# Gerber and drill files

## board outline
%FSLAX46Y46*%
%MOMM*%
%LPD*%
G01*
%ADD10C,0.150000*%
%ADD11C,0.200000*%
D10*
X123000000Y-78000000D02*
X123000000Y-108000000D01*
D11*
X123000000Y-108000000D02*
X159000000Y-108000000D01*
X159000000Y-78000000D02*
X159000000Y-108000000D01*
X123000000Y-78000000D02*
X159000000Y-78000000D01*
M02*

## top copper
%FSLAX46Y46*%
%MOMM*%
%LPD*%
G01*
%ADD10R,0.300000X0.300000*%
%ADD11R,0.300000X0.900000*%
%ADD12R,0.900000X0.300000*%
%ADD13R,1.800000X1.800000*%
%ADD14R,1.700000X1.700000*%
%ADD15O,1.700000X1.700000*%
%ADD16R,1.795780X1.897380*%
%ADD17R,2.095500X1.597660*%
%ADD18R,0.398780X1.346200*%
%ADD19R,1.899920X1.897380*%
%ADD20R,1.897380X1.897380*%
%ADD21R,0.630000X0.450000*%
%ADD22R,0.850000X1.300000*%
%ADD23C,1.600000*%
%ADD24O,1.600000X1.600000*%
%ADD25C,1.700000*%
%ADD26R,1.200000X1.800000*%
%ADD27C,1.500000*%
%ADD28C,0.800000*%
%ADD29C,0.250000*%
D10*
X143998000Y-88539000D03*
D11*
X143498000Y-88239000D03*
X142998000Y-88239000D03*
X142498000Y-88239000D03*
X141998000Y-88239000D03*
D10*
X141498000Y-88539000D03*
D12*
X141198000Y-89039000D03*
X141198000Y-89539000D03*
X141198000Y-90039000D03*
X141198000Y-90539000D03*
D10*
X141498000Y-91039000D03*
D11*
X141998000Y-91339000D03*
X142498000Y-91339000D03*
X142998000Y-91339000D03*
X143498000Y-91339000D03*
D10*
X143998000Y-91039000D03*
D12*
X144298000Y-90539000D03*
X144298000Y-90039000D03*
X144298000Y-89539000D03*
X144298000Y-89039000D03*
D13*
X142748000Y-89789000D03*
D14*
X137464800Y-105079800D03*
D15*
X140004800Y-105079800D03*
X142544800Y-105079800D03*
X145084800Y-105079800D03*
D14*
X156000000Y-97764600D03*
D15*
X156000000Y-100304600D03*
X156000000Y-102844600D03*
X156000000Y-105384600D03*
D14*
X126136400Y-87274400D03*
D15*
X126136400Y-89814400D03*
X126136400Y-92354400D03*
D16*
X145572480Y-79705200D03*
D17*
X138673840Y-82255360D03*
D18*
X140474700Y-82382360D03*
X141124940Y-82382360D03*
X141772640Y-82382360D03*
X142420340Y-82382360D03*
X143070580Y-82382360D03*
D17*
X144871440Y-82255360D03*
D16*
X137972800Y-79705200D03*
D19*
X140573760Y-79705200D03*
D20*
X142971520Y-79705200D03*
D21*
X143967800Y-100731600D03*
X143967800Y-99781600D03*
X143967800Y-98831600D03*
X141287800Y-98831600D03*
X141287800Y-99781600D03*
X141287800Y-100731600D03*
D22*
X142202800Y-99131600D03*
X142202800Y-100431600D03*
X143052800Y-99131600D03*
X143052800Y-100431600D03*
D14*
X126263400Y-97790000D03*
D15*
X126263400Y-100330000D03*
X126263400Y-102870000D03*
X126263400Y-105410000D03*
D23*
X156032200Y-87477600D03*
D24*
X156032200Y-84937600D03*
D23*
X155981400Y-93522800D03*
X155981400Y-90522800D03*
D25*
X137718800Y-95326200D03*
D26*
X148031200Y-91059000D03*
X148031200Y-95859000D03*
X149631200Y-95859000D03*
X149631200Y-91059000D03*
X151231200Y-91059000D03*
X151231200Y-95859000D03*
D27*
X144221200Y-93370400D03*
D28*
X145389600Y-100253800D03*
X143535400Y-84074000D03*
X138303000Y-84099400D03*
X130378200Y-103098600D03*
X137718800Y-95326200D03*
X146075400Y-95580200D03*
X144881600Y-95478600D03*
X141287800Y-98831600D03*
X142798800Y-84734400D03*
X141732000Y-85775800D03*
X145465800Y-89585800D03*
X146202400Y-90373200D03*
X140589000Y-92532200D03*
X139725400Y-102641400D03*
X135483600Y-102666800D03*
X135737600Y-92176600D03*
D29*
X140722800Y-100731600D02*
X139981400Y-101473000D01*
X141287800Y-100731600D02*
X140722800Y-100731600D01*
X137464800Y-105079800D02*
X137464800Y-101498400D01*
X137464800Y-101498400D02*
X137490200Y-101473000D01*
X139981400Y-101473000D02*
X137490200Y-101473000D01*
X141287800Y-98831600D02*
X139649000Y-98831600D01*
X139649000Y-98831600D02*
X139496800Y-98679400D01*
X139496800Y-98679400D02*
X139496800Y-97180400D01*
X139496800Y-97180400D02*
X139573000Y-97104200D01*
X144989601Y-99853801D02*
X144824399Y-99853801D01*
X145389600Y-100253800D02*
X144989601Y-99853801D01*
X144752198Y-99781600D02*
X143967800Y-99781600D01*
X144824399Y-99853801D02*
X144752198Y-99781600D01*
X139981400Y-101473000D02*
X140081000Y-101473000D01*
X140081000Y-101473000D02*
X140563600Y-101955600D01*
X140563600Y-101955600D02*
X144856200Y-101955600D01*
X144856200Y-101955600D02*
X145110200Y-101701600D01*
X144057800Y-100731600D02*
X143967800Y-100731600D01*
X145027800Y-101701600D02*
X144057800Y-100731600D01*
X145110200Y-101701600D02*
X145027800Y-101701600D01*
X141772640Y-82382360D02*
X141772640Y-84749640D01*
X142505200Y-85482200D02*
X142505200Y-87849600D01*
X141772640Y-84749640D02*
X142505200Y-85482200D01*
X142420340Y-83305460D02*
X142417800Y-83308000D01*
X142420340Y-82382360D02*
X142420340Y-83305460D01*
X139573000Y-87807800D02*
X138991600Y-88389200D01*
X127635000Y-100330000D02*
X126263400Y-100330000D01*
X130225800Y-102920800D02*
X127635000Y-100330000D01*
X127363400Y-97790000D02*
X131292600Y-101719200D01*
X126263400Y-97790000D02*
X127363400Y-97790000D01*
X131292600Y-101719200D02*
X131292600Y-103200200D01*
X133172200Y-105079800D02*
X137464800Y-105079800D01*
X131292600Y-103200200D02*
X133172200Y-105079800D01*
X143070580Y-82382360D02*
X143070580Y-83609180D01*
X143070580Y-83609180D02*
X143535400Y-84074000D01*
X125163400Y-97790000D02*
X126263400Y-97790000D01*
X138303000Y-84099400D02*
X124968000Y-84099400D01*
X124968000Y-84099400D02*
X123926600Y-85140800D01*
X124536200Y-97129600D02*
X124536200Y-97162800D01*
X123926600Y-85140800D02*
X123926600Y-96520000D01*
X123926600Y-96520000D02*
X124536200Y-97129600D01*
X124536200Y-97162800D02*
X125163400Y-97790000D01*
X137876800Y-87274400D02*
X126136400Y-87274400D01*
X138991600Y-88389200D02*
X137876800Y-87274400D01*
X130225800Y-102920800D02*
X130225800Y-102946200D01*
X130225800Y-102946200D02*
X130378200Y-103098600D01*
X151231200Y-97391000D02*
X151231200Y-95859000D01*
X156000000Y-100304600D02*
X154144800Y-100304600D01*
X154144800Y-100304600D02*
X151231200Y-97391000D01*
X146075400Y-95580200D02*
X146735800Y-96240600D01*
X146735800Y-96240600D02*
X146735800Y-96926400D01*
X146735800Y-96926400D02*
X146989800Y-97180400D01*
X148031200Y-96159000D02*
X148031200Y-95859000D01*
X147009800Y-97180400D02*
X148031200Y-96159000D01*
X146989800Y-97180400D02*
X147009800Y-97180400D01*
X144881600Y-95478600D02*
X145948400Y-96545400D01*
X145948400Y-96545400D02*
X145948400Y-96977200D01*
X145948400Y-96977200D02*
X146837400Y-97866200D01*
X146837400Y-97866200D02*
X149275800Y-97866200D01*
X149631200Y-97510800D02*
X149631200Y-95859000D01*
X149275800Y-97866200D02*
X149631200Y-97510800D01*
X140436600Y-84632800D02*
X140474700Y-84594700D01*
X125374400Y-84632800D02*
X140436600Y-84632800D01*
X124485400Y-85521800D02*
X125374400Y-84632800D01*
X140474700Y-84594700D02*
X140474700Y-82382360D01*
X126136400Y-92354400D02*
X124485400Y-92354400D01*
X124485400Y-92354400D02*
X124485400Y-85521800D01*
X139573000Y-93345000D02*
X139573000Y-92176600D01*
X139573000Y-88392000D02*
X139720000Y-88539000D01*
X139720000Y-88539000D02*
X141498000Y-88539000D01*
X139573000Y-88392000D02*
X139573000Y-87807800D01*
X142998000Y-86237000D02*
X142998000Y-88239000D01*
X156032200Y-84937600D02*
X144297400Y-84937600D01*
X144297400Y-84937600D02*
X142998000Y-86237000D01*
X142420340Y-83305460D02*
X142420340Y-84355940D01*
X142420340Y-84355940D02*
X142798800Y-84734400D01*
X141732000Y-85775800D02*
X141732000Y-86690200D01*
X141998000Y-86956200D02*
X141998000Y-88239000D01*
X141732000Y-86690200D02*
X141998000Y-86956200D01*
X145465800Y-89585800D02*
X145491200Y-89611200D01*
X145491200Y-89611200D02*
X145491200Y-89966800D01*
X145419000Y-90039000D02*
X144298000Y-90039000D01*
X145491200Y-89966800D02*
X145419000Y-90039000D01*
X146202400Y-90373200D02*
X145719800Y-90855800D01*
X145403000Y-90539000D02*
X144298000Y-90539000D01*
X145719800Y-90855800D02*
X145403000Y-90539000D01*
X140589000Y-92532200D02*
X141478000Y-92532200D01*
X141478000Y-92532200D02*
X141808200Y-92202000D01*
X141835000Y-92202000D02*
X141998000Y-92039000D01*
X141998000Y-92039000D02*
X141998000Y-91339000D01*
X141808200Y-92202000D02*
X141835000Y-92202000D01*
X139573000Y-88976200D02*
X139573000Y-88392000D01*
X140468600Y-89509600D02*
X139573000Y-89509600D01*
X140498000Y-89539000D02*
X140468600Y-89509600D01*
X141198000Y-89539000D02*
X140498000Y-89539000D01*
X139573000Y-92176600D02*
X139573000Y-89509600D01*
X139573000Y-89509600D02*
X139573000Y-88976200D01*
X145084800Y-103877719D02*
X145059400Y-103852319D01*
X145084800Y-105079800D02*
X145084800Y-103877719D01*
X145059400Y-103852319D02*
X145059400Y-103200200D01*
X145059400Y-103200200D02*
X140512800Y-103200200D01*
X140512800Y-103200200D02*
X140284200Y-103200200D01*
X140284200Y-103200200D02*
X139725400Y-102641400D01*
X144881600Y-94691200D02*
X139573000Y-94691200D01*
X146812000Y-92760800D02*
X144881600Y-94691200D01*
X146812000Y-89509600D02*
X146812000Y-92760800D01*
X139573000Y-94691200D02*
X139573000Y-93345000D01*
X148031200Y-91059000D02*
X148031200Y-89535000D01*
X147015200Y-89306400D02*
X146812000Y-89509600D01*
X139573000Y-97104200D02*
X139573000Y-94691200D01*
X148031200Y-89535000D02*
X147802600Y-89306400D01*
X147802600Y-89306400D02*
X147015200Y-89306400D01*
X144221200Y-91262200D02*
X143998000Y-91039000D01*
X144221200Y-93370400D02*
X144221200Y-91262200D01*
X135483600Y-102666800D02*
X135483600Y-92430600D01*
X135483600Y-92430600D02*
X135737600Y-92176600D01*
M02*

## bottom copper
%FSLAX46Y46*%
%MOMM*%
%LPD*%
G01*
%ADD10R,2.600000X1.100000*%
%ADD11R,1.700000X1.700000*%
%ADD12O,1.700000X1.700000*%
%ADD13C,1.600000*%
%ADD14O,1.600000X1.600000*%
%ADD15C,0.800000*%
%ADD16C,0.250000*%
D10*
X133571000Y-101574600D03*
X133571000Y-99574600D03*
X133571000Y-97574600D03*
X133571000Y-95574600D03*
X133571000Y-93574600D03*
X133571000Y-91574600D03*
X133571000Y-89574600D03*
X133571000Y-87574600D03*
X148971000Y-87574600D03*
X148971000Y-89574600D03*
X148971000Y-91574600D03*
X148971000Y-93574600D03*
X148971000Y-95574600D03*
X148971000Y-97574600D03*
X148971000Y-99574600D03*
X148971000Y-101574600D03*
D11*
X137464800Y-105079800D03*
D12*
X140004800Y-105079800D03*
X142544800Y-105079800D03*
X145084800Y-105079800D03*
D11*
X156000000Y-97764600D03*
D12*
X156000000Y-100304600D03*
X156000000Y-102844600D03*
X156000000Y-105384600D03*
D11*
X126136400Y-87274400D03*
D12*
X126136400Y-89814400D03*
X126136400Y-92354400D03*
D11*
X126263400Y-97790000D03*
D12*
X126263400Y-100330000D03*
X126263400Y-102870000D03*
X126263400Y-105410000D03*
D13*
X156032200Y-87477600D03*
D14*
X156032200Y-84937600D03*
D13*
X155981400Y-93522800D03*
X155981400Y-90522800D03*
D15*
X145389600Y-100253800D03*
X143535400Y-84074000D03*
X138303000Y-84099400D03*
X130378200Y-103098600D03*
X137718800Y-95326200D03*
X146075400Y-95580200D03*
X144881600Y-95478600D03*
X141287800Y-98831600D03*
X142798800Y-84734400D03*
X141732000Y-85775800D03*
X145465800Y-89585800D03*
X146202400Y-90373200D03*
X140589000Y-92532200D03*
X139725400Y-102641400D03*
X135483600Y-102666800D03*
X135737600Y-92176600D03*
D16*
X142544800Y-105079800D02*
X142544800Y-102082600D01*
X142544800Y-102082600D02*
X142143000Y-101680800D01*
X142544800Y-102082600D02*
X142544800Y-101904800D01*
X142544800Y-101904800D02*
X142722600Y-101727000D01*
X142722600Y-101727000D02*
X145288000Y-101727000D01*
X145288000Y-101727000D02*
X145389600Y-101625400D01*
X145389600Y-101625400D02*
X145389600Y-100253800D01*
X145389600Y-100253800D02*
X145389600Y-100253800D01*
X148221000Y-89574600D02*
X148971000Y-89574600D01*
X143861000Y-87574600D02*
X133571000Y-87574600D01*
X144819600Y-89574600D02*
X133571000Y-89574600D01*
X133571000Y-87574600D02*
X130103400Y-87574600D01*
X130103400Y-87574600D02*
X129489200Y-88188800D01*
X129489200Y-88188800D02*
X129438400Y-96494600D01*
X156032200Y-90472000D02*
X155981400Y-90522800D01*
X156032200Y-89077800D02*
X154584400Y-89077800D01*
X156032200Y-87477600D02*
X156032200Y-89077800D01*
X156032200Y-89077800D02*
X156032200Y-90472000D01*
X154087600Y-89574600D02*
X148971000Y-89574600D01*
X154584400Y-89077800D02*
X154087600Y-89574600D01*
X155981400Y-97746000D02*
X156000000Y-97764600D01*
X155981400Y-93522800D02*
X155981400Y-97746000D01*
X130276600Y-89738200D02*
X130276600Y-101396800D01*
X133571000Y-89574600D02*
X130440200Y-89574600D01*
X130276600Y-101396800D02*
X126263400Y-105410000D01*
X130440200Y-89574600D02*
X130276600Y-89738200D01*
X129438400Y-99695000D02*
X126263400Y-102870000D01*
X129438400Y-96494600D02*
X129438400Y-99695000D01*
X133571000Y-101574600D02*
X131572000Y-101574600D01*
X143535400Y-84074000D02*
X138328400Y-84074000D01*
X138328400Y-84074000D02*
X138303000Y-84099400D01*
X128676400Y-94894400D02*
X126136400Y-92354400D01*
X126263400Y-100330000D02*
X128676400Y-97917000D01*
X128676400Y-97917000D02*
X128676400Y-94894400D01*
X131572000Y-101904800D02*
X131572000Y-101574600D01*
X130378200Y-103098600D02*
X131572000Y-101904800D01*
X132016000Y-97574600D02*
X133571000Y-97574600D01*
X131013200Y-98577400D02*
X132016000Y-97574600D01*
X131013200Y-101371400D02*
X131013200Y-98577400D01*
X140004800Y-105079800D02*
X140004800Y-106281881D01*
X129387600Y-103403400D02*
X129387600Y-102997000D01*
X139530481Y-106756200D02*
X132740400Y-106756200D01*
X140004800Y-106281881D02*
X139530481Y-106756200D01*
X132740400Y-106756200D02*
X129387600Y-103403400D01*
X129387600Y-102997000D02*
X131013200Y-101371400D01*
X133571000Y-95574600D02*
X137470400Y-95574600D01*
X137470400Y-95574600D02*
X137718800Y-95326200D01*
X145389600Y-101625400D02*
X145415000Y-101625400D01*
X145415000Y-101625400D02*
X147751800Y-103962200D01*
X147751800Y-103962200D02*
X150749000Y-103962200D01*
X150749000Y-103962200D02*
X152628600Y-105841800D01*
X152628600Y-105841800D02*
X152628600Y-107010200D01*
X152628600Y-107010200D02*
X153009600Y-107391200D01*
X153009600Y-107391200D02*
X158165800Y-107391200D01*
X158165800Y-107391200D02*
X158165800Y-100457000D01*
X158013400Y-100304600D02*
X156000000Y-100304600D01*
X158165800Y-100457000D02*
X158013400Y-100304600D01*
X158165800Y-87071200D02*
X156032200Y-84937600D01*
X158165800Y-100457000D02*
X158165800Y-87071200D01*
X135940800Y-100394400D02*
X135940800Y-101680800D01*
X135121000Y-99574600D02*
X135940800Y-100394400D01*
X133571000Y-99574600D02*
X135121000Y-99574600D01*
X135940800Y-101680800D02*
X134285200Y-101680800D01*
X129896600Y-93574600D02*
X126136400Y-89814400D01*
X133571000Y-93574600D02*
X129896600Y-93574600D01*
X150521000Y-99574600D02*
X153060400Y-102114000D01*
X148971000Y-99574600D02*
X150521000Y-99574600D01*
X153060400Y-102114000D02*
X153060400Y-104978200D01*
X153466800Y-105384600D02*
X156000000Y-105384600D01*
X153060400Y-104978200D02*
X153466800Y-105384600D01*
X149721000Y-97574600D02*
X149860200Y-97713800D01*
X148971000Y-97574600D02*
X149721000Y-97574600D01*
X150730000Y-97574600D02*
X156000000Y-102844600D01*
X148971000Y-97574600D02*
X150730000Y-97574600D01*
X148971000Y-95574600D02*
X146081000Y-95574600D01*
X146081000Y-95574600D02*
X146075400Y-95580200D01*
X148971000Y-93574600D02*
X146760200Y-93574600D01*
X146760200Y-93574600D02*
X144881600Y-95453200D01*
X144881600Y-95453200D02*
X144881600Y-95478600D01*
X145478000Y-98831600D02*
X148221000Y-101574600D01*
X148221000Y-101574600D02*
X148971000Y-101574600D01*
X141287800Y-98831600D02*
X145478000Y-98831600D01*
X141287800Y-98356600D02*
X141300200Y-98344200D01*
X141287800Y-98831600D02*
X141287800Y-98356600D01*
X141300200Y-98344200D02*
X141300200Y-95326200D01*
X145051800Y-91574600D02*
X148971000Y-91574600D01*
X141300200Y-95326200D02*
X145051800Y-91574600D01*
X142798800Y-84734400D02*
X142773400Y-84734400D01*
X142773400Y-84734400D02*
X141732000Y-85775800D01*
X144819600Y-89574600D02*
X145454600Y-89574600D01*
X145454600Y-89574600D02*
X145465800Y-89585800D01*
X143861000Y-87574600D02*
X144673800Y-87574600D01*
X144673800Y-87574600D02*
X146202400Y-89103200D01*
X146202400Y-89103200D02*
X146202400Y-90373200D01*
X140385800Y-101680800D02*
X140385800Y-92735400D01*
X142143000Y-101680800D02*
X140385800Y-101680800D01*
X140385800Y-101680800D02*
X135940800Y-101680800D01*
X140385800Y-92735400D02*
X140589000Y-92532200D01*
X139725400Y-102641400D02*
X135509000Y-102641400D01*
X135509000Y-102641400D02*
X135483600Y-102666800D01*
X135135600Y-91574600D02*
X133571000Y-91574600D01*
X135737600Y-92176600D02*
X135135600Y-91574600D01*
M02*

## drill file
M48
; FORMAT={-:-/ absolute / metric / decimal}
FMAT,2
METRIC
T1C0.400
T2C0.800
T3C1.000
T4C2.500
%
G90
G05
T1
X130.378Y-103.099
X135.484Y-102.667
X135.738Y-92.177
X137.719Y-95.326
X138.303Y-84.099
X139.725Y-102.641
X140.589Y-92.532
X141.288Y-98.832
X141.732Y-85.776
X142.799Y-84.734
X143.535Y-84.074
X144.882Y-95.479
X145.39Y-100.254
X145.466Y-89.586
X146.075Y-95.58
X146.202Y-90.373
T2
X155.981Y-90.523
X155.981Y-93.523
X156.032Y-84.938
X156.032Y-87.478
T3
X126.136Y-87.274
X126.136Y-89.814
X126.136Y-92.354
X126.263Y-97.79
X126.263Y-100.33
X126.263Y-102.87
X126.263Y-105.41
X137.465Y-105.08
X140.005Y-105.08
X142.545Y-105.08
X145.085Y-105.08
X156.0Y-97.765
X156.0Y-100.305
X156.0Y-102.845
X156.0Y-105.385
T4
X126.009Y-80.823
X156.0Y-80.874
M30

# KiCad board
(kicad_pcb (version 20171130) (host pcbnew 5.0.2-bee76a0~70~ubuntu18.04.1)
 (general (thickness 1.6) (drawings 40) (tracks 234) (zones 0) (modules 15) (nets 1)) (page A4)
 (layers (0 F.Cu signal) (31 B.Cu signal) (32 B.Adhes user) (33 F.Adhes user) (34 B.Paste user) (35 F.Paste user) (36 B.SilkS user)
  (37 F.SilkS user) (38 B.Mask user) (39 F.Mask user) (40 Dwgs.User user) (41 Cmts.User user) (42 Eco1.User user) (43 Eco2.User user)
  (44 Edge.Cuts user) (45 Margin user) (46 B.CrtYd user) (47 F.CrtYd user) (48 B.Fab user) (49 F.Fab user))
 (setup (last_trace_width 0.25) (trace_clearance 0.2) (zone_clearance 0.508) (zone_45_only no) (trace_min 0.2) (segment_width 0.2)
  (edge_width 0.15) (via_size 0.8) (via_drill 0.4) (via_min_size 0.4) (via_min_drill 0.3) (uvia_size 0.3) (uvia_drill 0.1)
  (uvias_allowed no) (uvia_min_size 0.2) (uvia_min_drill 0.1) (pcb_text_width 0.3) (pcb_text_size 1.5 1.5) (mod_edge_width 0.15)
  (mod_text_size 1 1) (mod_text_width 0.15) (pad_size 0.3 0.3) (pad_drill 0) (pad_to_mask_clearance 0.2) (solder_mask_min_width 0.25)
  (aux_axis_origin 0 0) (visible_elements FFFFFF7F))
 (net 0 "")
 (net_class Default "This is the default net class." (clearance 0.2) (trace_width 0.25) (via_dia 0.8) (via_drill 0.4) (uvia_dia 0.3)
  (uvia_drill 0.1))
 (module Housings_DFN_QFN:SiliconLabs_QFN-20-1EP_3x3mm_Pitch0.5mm (layer F.Cu) (at 142.748 89.789 270)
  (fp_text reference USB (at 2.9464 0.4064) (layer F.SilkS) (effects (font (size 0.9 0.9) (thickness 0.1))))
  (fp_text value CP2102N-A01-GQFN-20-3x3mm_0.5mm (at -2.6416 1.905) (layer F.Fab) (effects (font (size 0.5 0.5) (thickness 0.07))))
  (pad 1 smd rect (at -1.25 -1.25 270) (size 0.3 0.3) (layers F.Cu F.Paste F.Mask))
  (pad 2 smd rect (at -1.55 -0.75 270) (size 0.9 0.3) (layers F.Cu F.Paste F.Mask))
  (pad GND smd rect (at -1.55 -0.25 270) (size 0.9 0.3) (layers F.Cu F.Paste F.Mask))
  (pad D+ smd rect (at -1.55 0.25 270) (size 0.9 0.3) (layers F.Cu F.Paste F.Mask))
  (pad D- smd rect (at -1.55 0.75 270) (size 0.9 0.3) (layers F.Cu F.Paste F.Mask))
  (pad +3.3 smd rect (at -1.25 1.25 270) (size 0.3 0.3) (layers F.Cu F.Paste F.Mask))
  (pad VREGIN smd rect (at -0.75 1.55) (size 0.9 0.3) (layers F.Cu F.Paste F.Mask))
  (pad VBUS smd rect (at -0.25 1.55) (size 0.9 0.3) (layers F.Cu F.Paste F.Mask))
  (pad 9 smd rect (at 0.25 1.55) (size 0.9 0.3) (layers F.Cu F.Paste F.Mask))
  (pad 10 smd rect (at 0.75 1.55) (size 0.9 0.3) (layers F.Cu F.Paste F.Mask))
  (pad 11 smd rect (at 1.25 1.25 270) (size 0.3 0.3) (layers F.Cu F.Paste F.Mask))
  (pad GND smd rect (at 1.55 0.75 270) (size 0.9 0.3) (layers F.Cu F.Paste F.Mask))
  (pad 13 smd rect (at 1.55 0.25 270) (size 0.9 0.3) (layers F.Cu F.Paste F.Mask))
  (pad 14 smd rect (at 1.55 -0.25 270) (size 0.9 0.3) (layers F.Cu F.Paste F.Mask))
  (pad 15 smd rect (at 1.55 -0.75 270) (size 0.9 0.3) (layers F.Cu F.Paste F.Mask))
  (pad 16 smd rect (at 1.25 -1.25 270) (size 0.3 0.3) (layers F.Cu F.Paste F.Mask))
  (pad RX smd rect (at 0.75 -1.55) (size 0.9 0.3) (layers F.Cu F.Paste F.Mask))
  (pad TX smd rect (at 0.25 -1.55) (size 0.9 0.3) (layers F.Cu F.Paste F.Mask))
  (pad 19 smd rect (at -0.25 -1.55) (size 0.9 0.3) (layers F.Cu F.Paste F.Mask))
  (pad 20 smd rect (at -0.75 -1.55) (size 0.9 0.3) (layers F.Cu F.Paste F.Mask))
  (pad 21 smd rect (at 0 0 270) (size 1.8 1.8) (layers F.Cu F.Mask))
  (pad "" smd rect (at -0.45 -0.45 270) (size 0.54 0.54) (layers F.Paste))
  (pad "" smd rect (at -0.45 0.45 270) (size 0.54 0.54) (layers F.Paste))
  (pad "" smd rect (at 0.45 -0.45 270) (size 0.54 0.54) (layers F.Paste))
  (pad "" smd rect (at 0.45 0.45 270) (size 0.54 0.54) (layers F.Paste)))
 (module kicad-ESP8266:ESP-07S (layer B.Cu) (at 141.271 94.5746)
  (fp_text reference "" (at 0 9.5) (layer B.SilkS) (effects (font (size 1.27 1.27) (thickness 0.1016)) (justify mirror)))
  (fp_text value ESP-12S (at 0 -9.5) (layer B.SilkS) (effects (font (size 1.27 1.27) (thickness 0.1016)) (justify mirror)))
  (pad GND smd rect (at -7.7 7) (size 2.6 1.1) (layers B.Cu B.Paste B.Mask))
  (pad IO15 smd rect (at -7.7 5) (size 2.6 1.1) (layers B.Cu B.Paste B.Mask))
  (pad IO2 smd rect (at -7.7 3) (size 2.6 1.1) (layers B.Cu B.Paste B.Mask))
  (pad IO0 smd rect (at -7.7 1) (size 2.6 1.1) (layers B.Cu B.Paste B.Mask))
  (pad IO4 smd rect (at -7.7 -1) (size 2.6 1.1) (layers B.Cu B.Paste B.Mask))
  (pad IO5 smd rect (at -7.7 -3) (size 2.6 1.1) (layers B.Cu B.Paste B.Mask))
  (pad RX smd rect (at -7.7 -5) (size 2.6 1.1) (layers B.Cu B.Paste B.Mask))
  (pad TX smd rect (at -7.7 -7) (size 2.6 1.1) (layers B.Cu B.Paste B.Mask))
  (pad RST smd rect (at 7.7 -7) (size 2.6 1.1) (layers B.Cu B.Paste B.Mask))
  (pad ADC smd rect (at 7.7 -5) (size 2.6 1.1) (layers B.Cu B.Paste B.Mask))
  (pad EN smd rect (at 7.7 -3) (size 2.6 1.1) (layers B.Cu B.Paste B.Mask))
  (pad IO16 smd rect (at 7.7 -1) (size 2.6 1.1) (layers B.Cu B.Paste B.Mask))
  (pad IO14 smd rect (at 7.7 1) (size 2.6 1.1) (layers B.Cu B.Paste B.Mask))
  (pad IO12 smd rect (at 7.7 3) (size 2.6 1.1) (layers B.Cu B.Paste B.Mask))
  (pad IO13 smd rect (at 7.7 5) (size 2.6 1.1) (layers B.Cu B.Paste B.Mask))
  (pad VCC smd rect (at 7.7 7) (size 2.6 1.1) (layers B.Cu B.Paste B.Mask)))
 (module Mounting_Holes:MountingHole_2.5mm (layer F.Cu) (at 126.0094 80.8228)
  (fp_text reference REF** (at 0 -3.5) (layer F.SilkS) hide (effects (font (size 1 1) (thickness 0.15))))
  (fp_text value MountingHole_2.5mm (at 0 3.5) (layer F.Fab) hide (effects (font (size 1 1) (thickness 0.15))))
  (pad 1 np_thru_hole circle (at 0 0) (size 2.5 2.5) (drill 2.5) (layers *.Cu *.Mask)))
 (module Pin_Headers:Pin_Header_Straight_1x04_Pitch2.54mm (layer F.Cu) (at 137.4648 105.0798 90)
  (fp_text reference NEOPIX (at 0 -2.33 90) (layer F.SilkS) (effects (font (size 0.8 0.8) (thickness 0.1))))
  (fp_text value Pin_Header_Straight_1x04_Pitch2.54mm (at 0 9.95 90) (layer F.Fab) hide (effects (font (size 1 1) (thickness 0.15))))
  (pad +V thru_hole rect (at 0 0 90) (size 1.7 1.7) (drill 1) (layers *.Cu *.Mask))
  (pad 2 thru_hole oval (at 0 2.54 90) (size 1.7 1.7) (drill 1) (layers *.Cu *.Mask))
  (pad GND thru_hole oval (at 0 5.08 90) (size 1.7 1.7) (drill 1) (layers *.Cu *.Mask))
  (pad 4 thru_hole oval (at 0 7.62 90) (size 1.7 1.7) (drill 1) (layers *.Cu *.Mask)))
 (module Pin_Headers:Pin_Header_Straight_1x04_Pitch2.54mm (layer F.Cu) (at 156 97.7646)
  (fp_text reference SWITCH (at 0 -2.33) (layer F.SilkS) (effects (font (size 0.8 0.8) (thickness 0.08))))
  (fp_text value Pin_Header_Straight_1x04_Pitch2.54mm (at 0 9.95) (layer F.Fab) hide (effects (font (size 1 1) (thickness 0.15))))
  (pad +3.3 thru_hole rect (at 0 0) (size 1.7 1.7) (drill 1) (layers *.Cu *.Mask))
  (pad GND thru_hole oval (at 0 2.54) (size 1.7 1.7) (drill 1) (layers *.Cu *.Mask))
  (pad 3 thru_hole oval (at 0 5.08) (size 1.7 1.7) (drill 1) (layers *.Cu *.Mask))
  (pad 4 thru_hole oval (at 0 7.62) (size 1.7 1.7) (drill 1) (layers *.Cu *.Mask)))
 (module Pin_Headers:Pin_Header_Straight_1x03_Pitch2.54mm (layer F.Cu) (at 126.1364 87.2744)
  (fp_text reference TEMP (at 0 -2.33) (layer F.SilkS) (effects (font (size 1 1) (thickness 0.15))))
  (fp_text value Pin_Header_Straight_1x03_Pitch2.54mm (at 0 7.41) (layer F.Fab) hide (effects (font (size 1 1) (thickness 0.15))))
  (pad +3.3 thru_hole rect (at 0 0) (size 1.7 1.7) (drill 1) (layers *.Cu *.Mask))
  (pad 2 thru_hole oval (at 0 2.54) (size 1.7 1.7) (drill 1) (layers *.Cu *.Mask))
  (pad GND thru_hole oval (at 0 5.08) (size 1.7 1.7) (drill 1) (layers *.Cu *.Mask)))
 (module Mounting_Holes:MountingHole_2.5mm (layer F.Cu) (at 155.9814 80.8736)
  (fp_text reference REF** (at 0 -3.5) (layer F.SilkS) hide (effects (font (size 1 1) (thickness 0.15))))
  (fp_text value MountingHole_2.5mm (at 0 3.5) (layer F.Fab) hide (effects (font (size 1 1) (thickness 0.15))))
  (pad "" np_thru_hole circle (at 0.0186 0) (size 2.5 2.5) (drill 2.5) (layers *.Cu *.Mask)))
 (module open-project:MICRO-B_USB (layer F.Cu) (at 141.77264 78.2574 180)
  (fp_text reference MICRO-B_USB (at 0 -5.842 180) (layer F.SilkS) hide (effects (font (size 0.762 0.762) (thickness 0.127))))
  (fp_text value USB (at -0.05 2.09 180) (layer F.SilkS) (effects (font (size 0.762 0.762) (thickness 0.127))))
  (pad "" smd rect (at -3.79984 -1.4478 180) (size 1.79578 1.89738) (layers F.Cu F.Paste F.Mask))
  (pad "" smd rect (at 3.0988 -3.99796 180) (size 2.0955 1.59766) (layers F.Cu F.Paste F.Mask))
  (pad GND smd rect (at 1.29794 -4.12496 180) (size 0.39878 1.3462) (layers F.Cu F.Paste F.Mask) (clearance 0.2032))
  (pad ID smd rect (at 0.6477 -4.12496 180) (size 0.39878 1.3462) (layers F.Cu F.Paste F.Mask) (clearance 0.2032))
  (pad D+ smd rect (at 0 -4.12496 180) (size 0.39878 1.3462) (layers F.Cu F.Paste F.Mask) (clearance 0.2032))
  (pad D- smd rect (at -0.6477 -4.12496 180) (size 0.39878 1.3462) (layers F.Cu F.Paste F.Mask) (clearance 0.2032))
  (pad +5V smd rect (at -1.29794 -4.12496 180) (size 0.39878 1.3462) (layers F.Cu F.Paste F.Mask) (clearance 0.2032))
  (pad "" smd rect (at -3.0988 -3.99796 180) (size 2.0955 1.59766) (layers F.Cu F.Paste F.Mask))
  (pad "" smd rect (at 3.79984 -1.4478 180) (size 1.79578 1.89738) (layers F.Cu F.Paste F.Mask))
  (pad "" smd rect (at 1.19888 -1.4478 180) (size 1.89992 1.89738) (layers F.Cu F.Paste F.Mask))
  (pad "" smd rect (at -1.19888 -1.4478 180) (size 1.89738 1.89738) (layers F.Cu F.Paste F.Mask)))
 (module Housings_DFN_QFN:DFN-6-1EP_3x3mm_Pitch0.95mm (layer F.Cu) (at 142.6278 99.7816 180)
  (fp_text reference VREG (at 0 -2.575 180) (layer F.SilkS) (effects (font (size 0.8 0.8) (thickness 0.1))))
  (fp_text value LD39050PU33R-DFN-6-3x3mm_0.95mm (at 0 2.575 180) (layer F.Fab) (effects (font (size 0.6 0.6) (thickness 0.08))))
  (pad EN smd rect (at -1.34 -0.95 180) (size 0.63 0.45) (layers F.Cu F.Paste F.Mask))
  (pad GND smd rect (at -1.34 0 180) (size 0.63 0.45) (layers F.Cu F.Paste F.Mask))
  (pad PG smd rect (at -1.34 0.95 180) (size 0.63 0.45) (layers F.Cu F.Paste F.Mask))
  (pad VOUT smd rect (at 1.34 0.95 180) (size 0.63 0.45) (layers F.Cu F.Paste F.Mask))
  (pad 5 smd rect (at 1.34 0 180) (size 0.63 0.45) (layers F.Cu F.Paste F.Mask))
  (pad VIN smd rect (at 1.34 -0.95 180) (size 0.63 0.45) (layers F.Cu F.Paste F.Mask))
  (pad 7 smd rect (at 0.425 0.65 180) (size 0.85 1.3) (layers F.Cu F.Paste F.Mask) (solder_paste_margin_ratio -0.2))
  (pad 7 smd rect (at 0.425 -0.65 180) (size 0.85 1.3) (layers F.Cu F.Paste F.Mask) (solder_paste_margin_ratio -0.2))
  (pad 7 smd rect (at -0.425 0.65 180) (size 0.85 1.3) (layers F.Cu F.Paste F.Mask) (solder_paste_margin_ratio -0.2))
  (pad 7 smd rect (at -0.425 -0.65 180) (size 0.85 1.3) (layers F.Cu F.Paste F.Mask) (solder_paste_margin_ratio -0.2)))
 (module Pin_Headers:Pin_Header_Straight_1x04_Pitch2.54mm (layer F.Cu) (at 126.2634 97.79)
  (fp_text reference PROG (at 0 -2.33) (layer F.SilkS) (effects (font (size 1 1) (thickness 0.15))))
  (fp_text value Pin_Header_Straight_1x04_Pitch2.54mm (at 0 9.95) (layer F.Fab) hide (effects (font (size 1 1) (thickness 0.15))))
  (pad +v thru_hole rect (at 0 0) (size 1.7 1.7) (drill 1) (layers *.Cu *.Mask))
  (pad GND thru_hole oval (at 0 2.54) (size 1.7 1.7) (drill 1) (layers *.Cu *.Mask))
  (pad TX thru_hole oval (at 0 5.08) (size 1.7 1.7) (drill 1) (layers *.Cu *.Mask))
  (pad RX thru_hole oval (at 0 7.62) (size 1.7 1.7) (drill 1) (layers *.Cu *.Mask)))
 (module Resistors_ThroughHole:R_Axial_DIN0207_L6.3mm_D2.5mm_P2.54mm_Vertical (layer F.Cu) (at 156.0322 87.4776 90)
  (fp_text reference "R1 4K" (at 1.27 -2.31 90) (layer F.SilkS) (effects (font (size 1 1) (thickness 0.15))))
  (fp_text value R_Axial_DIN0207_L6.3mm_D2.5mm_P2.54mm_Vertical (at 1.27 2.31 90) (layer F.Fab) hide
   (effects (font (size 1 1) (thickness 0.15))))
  (pad 1 thru_hole circle (at 0 0 90) (size 1.6 1.6) (drill 0.8) (layers *.Cu *.Mask))
  (pad GND thru_hole oval (at 2.54 0 90) (size 1.6 1.6) (drill 0.8) (layers *.Cu *.Mask)))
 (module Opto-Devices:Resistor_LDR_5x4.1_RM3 (layer F.Cu) (at 155.9814 93.5228 90)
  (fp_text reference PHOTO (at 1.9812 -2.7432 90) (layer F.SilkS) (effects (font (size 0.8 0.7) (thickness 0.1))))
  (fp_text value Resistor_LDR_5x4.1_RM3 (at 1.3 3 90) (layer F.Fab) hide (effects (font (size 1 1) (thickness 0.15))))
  (pad 1 thru_hole circle (at 0 0 90) (size 1.6 1.6) (drill 0.8) (layers *.Cu *.Mask))
  (pad 2 thru_hole circle (at 3 0 90) (size 1.6 1.6) (drill 0.8) (layers *.Cu *.Mask)))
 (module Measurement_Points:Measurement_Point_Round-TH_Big (layer F.Cu) (at 137.7188 95.3262)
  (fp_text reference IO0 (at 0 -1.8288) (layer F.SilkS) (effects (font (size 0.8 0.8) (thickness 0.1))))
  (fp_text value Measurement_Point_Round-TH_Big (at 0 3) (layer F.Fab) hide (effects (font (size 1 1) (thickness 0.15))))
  (pad 1 smd circle (at 0 0) (size 1.7 1.7) (layers F.Cu F.Paste F.Mask)))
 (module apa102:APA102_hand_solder (layer F.Cu) (at 149.6312 93.459) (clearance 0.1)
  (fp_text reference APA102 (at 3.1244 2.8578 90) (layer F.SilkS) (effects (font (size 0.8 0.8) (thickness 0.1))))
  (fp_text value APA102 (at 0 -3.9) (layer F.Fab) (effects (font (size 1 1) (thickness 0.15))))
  (pad VCC smd rect (at -1.6 -2.4 90) (size 1.8 1.2) (layers F.Cu F.Paste F.Mask))
  (pad IN-DA smd rect (at -1.6 2.4 90) (size 1.8 1.2) (layers F.Cu F.Paste F.Mask))
  (pad IN-CL smd rect (at 0 2.4 90) (size 1.8 1.2) (layers F.Cu F.Paste F.Mask))
  (pad OUT-CLK smd rect (at 0 -2.4 90) (size 1.8 1.2) (layers F.Cu F.Paste F.Mask))
  (pad OUT-DA smd rect (at 1.6 -2.4 90) (size 1.8 1.2) (layers F.Cu F.Paste F.Mask))
  (pad GND smd rect (at 1.6 2.4 90) (size 1.8 1.2) (layers F.Cu F.Paste F.Mask)))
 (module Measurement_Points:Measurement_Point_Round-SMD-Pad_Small (layer F.Cu) (at 144.2212 93.3704)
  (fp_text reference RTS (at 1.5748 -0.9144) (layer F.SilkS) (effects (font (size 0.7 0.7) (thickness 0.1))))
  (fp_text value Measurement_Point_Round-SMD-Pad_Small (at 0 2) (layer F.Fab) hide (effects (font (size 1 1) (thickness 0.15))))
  (pad 1 smd circle (at 0 0) (size 1.5 1.5) (layers F.Cu F.Mask)))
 (gr_line (start 123 78) (end 123 108) (layer Edge.Cuts) (width 0.15))
 (gr_line (start 123 108) (end 159 108) (layer Edge.Cuts) (width 0.2))
 (gr_line (start 159 78) (end 159 108) (layer Edge.Cuts) (width 0.2))
 (gr_line (start 123 78) (end 159 78) (layer Edge.Cuts) (width 0.2))
 (segment (start 140.7228 100.7316) (end 139.9814 101.473) (width 0.25) (layer F.Cu) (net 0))
 (segment (start 141.2878 100.7316) (end 140.7228 100.7316) (width 0.25) (layer F.Cu) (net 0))
 (segment (start 137.4648 105.0798) (end 137.4648 101.4984) (width 0.25) (layer F.Cu) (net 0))
 (segment (start 137.4648 101.4984) (end 137.4902 101.473) (width 0.25) (layer F.Cu) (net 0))
 (segment (start 139.9814 101.473) (end 137.4902 101.473) (width 0.25) (layer F.Cu) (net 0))
 (segment (start 141.2878 98.8316) (end 139.649 98.8316) (width 0.25) (layer F.Cu) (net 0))
 (segment (start 139.649 98.8316) (end 139.4968 98.6794) (width 0.25) (layer F.Cu) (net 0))
 (segment (start 139.4968 98.6794) (end 139.4968 97.1804) (width 0.25) (layer F.Cu) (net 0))
 (segment (start 139.4968 97.1804) (end 139.573 97.1042) (width 0.25) (layer F.Cu) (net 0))
 (segment (start 142.5448 105.0798) (end 142.5448 102.0826) (width 0.25) (layer B.Cu) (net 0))
 (segment (start 142.5448 102.0826) (end 142.143 101.6808) (width 0.25) (layer B.Cu) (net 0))
 (segment (start 142.5448 102.0826) (end 142.5448 101.9048) (width 0.25) (layer B.Cu) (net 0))
 (segment (start 142.5448 101.9048) (end 142.7226 101.727) (width 0.25) (layer B.Cu) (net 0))
 (segment (start 142.7226 101.727) (end 145.288 101.727) (width 0.25) (layer B.Cu) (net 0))
 (segment (start 145.288 101.727) (end 145.3896 101.6254) (width 0.25) (layer B.Cu) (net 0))
 (segment (start 145.3896 101.6254) (end 145.3896 100.2538) (width 0.25) (layer B.Cu) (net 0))
 (segment (start 145.3896 100.2538) (end 145.3896 100.2538) (width 0.25) (layer B.Cu) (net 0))
 (via (at 145.3896 100.2538) (size 0.8) (drill 0.4) (layers F.Cu B.Cu) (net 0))
 (segment (start 144.989601 99.853801) (end 144.824399 99.853801) (width 0.25) (layer F.Cu) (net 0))
 (segment (start 145.3896 100.2538) (end 144.989601 99.853801) (width 0.25) (layer F.Cu) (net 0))
 (segment (start 144.752198 99.7816) (end 143.9678 99.7816) (width 0.25) (layer F.Cu) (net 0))
 (segment (start 144.824399 99.853801) (end 144.752198 99.7816) (width 0.25) (layer F.Cu) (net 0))
 (segment (start 139.9814 101.473) (end 140.081 101.473) (width 0.25) (layer F.Cu) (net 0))
 (segment (start 140.081 101.473) (end 140.5636 101.9556) (width 0.25) (layer F.Cu) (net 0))
 (segment (start 140.5636 101.9556) (end 144.8562 101.9556) (width 0.25) (layer F.Cu) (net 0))
 (segment (start 144.8562 101.9556) (end 145.1102 101.7016) (width 0.25) (layer F.Cu) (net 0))
 (segment (start 144.0578 100.7316) (end 143.9678 100.7316) (width 0.25) (layer F.Cu) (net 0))
 (segment (start 145.0278 101.7016) (end 144.0578 100.7316) (width 0.25) (layer F.Cu) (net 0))
 (segment (start 145.1102 101.7016) (end 145.0278 101.7016) (width 0.25) (layer F.Cu) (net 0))
 (segment (start 141.77264 82.38236) (end 141.77264 84.74964) (width 0.25) (layer F.Cu) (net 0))
 (segment (start 142.5052 85.4822) (end 142.5052 87.8496) (width 0.25) (layer F.Cu) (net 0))
 (segment (start 141.77264 84.74964) (end 142.5052 85.4822) (width 0.25) (layer F.Cu) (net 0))
 (segment (start 142.42034 83.30546) (end 142.4178 83.308) (width 0.25) (layer F.Cu) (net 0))
 (segment (start 142.42034 82.38236) (end 142.42034 83.30546) (width 0.25) (layer F.Cu) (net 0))
 (segment (start 139.573 87.8078) (end 138.9916 88.3892) (width 0.25) (layer F.Cu) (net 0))
 (segment (start 148.221 89.5746) (end 148.971 89.5746) (width 0.25) (layer B.Cu) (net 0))
 (segment (start 143.861 87.5746) (end 133.571 87.5746) (width 0.25) (layer B.Cu) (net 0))
 (segment (start 144.8196 89.5746) (end 133.571 89.5746) (width 0.25) (layer B.Cu) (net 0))
 (segment (start 133.571 87.5746) (end 130.1034 87.5746) (width 0.25) (layer B.Cu) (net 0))
 (segment (start 130.1034 87.5746) (end 129.4892 88.1888) (width 0.25) (layer B.Cu) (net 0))
 (segment (start 129.4892 88.1888) (end 129.4384 96.4946) (width 0.25) (layer B.Cu) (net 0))
 (segment (start 156.0322 90.472) (end 155.9814 90.5228) (width 0.25) (layer B.Cu) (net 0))
 (segment (start 156.0322 89.0778) (end 154.5844 89.0778) (width 0.25) (layer B.Cu) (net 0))
 (segment (start 156.0322 87.4776) (end 156.0322 89.0778) (width 0.25) (layer B.Cu) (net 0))
 (segment (start 156.0322 89.0778) (end 156.0322 90.472) (width 0.25) (layer B.Cu) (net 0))
 (segment (start 154.0876 89.5746) (end 148.971 89.5746) (width 0.25) (layer B.Cu) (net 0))
 (segment (start 154.5844 89.0778) (end 154.0876 89.5746) (width 0.25) (layer B.Cu) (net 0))
 (segment (start 155.9814 97.746) (end 156 97.7646) (width 0.25) (layer B.Cu) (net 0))
 (segment (start 155.9814 93.5228) (end 155.9814 97.746) (width 0.25) (layer B.Cu) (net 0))
 (segment (start 130.2766 89.7382) (end 130.2766 101.3968) (width 0.25) (layer B.Cu) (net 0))
 (segment (start 133.571 89.5746) (end 130.4402 89.5746) (width 0.25) (layer B.Cu) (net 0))
 (segment (start 130.2766 101.3968) (end 126.2634 105.41) (width 0.25) (layer B.Cu) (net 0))
 (segment (start 130.4402 89.5746) (end 130.2766 89.7382) (width 0.25) (layer B.Cu) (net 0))
 (segment (start 129.4384 99.695) (end 126.2634 102.87) (width 0.25) (layer B.Cu) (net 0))
 (segment (start 129.4384 96.4946) (end 129.4384 99.695) (width 0.25) (layer B.Cu) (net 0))
 (segment (start 133.571 101.5746) (end 131.572 101.5746) (width 0.25) (layer B.Cu) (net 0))
 (segment (start 127.635 100.33) (end 126.2634 100.33) (width 0.25) (layer F.Cu) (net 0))
 (segment (start 130.2258 102.9208) (end 127.635 100.33) (width 0.25) (layer F.Cu) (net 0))
 (segment (start 127.3634 97.79) (end 131.2926 101.7192) (width 0.25) (layer F.Cu) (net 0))
 (segment (start 126.2634 97.79) (end 127.3634 97.79) (width 0.25) (layer F.Cu) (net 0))
 (segment (start 131.2926 101.7192) (end 131.2926 103.2002) (width 0.25) (layer F.Cu) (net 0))
 (segment (start 133.1722 105.0798) (end 137.4648 105.0798) (width 0.25) (layer F.Cu) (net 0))
 (segment (start 131.2926 103.2002) (end 133.1722 105.0798) (width 0.25) (layer F.Cu) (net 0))
 (via (at 143.5354 84.074) (size 0.8) (drill 0.4) (layers F.Cu B.Cu) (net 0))
 (segment (start 143.07058 82.38236) (end 143.07058 83.60918) (width 0.25) (layer F.Cu) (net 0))
 (segment (start 143.07058 83.60918) (end 143.5354 84.074) (width 0.25) (layer F.Cu) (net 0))
 (via (at 138.303 84.0994) (size 0.8) (drill 0.4) (layers F.Cu B.Cu) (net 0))
 (segment (start 143.5354 84.074) (end 138.3284 84.074) (width 0.25) (layer B.Cu) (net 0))
 (segment (start 138.3284 84.074) (end 138.303 84.0994) (width 0.25) (layer B.Cu) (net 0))
 (segment (start 125.1634 97.79) (end 126.2634 97.79) (width 0.25) (layer F.Cu) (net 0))
 (segment (start 138.303 84.0994) (end 124.968 84.0994) (width 0.25) (layer F.Cu) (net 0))
 (segment (start 124.968 84.0994) (end 123.9266 85.1408) (width 0.25) (layer F.Cu) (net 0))
 (segment (start 124.5362 97.1296) (end 124.5362 97.1628) (width 0.25) (layer F.Cu) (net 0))
 (segment (start 123.9266 85.1408) (end 123.9266 96.52) (width 0.25) (layer F.Cu) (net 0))
 (segment (start 123.9266 96.52) (end 124.5362 97.1296) (width 0.25) (layer F.Cu) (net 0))
 (segment (start 124.5362 97.1628) (end 125.1634 97.79) (width 0.25) (layer F.Cu) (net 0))
 (segment (start 137.8768 87.2744) (end 126.1364 87.2744) (width 0.25) (layer F.Cu) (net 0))
 (segment (start 138.9916 88.3892) (end 137.8768 87.2744) (width 0.25) (layer F.Cu) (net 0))
 (segment (start 128.6764 94.8944) (end 126.1364 92.3544) (width 0.25) (layer B.Cu) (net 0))
 (segment (start 126.2634 100.33) (end 128.6764 97.917) (width 0.25) (layer B.Cu) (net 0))
 (segment (start 128.6764 97.917) (end 128.6764 94.8944) (width 0.25) (layer B.Cu) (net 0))
 (via (at 130.3782 103.0986) (size 0.8) (drill 0.4) (layers F.Cu B.Cu) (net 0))
 (segment (start 130.2258 102.9208) (end 130.2258 102.9462) (width 0.25) (layer F.Cu) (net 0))
 (segment (start 130.2258 102.9462) (end 130.3782 103.0986) (width 0.25) (layer F.Cu) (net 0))
 (segment (start 131.572 101.9048) (end 131.572 101.5746) (width 0.25) (layer B.Cu) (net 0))
 (segment (start 130.3782 103.0986) (end 131.572 101.9048) (width 0.25) (layer B.Cu) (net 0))
 (segment (start 132.016 97.5746) (end 133.571 97.5746) (width 0.25) (layer B.Cu) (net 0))
 (segment (start 131.0132 98.5774) (end 132.016 97.5746) (width 0.25) (layer B.Cu) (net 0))
 (segment (start 131.0132 101.3714) (end 131.0132 98.5774) (width 0.25) (layer B.Cu) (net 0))
 (segment (start 140.0048 105.0798) (end 140.0048 106.281881) (width 0.25) (layer B.Cu) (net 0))
 (segment (start 129.3876 103.4034) (end 129.3876 102.997) (width 0.25) (layer B.Cu) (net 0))
 (segment (start 139.530481 106.7562) (end 132.7404 106.7562) (width 0.25) (layer B.Cu) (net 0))
 (segment (start 140.0048 106.281881) (end 139.530481 106.7562) (width 0.25) (layer B.Cu) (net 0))
 (segment (start 132.7404 106.7562) (end 129.3876 103.4034) (width 0.25) (layer B.Cu) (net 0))
 (segment (start 129.3876 102.997) (end 131.0132 101.3714) (width 0.25) (layer B.Cu) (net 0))
 (segment (start 133.571 95.5746) (end 137.4704 95.5746) (width 0.25) (layer B.Cu) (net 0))
 (via (at 137.7188 95.3262) (size 0.8) (drill 0.4) (layers F.Cu B.Cu) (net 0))
 (segment (start 137.4704 95.5746) (end 137.7188 95.3262) (width 0.25) (layer B.Cu) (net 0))
 (segment (start 145.3896 101.6254) (end 145.415 101.6254) (width 0.25) (layer B.Cu) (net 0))
 (segment (start 145.415 101.6254) (end 147.7518 103.9622) (width 0.25) (layer B.Cu) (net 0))
 (segment (start 147.7518 103.9622) (end 150.749 103.9622) (width 0.25) (layer B.Cu) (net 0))
 (segment (start 150.749 103.9622) (end 152.6286 105.8418) (width 0.25) (layer B.Cu) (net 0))
 (segment (start 152.6286 105.8418) (end 152.6286 107.0102) (width 0.25) (layer B.Cu) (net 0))
 (segment (start 152.6286 107.0102) (end 153.0096 107.3912) (width 0.25) (layer B.Cu) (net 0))
 (segment (start 153.0096 107.3912) (end 158.1658 107.3912) (width 0.25) (layer B.Cu) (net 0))
 (segment (start 158.1658 107.3912) (end 158.1658 100.457) (width 0.25) (layer B.Cu) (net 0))
 (segment (start 158.0134 100.3046) (end 156 100.3046) (width 0.25) (layer B.Cu) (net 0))
 (segment (start 158.1658 100.457) (end 158.0134 100.3046) (width 0.25) (layer B.Cu) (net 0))
 (segment (start 158.1658 87.0712) (end 156.0322 84.9376) (width 0.25) (layer B.Cu) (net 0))
 (segment (start 158.1658 100.457) (end 158.1658 87.0712) (width 0.25) (layer B.Cu) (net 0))
 (segment (start 135.9408 100.3944) (end 135.9408 101.6808) (width 0.25) (layer B.Cu) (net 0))
 (segment (start 135.121 99.5746) (end 135.9408 100.3944) (width 0.25) (layer B.Cu) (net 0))
 (segment (start 133.571 99.5746) (end 135.121 99.5746) (width 0.25) (layer B.Cu) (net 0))
 (segment (start 135.9408 101.6808) (end 134.2852 101.6808) (width 0.25) (layer B.Cu) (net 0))
 (segment (start 129.8966 93.5746) (end 126.1364 89.8144) (width 0.25) (layer B.Cu) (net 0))
 (segment (start 133.571 93.5746) (end 129.8966 93.5746) (width 0.25) (layer B.Cu) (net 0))
 (segment (start 150.521 99.5746) (end 153.0604 102.114) (width 0.25) (layer B.Cu) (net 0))
 (segment (start 148.971 99.5746) (end 150.521 99.5746) (width 0.25) (layer B.Cu) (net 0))
 (segment (start 153.0604 102.114) (end 153.0604 104.9782) (width 0.25) (layer B.Cu) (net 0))
 (segment (start 153.4668 105.3846) (end 156 105.3846) (width 0.25) (layer B.Cu) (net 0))
 (segment (start 153.0604 104.9782) (end 153.4668 105.3846) (width 0.25) (layer B.Cu) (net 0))
 (segment (start 149.721 97.5746) (end 149.8602 97.7138) (width 0.25) (layer B.Cu) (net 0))
 (segment (start 148.971 97.5746) (end 149.721 97.5746) (width 0.25) (layer B.Cu) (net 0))
 (segment (start 150.73 97.5746) (end 156 102.8446) (width 0.25) (layer B.Cu) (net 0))
 (segment (start 148.971 97.5746) (end 150.73 97.5746) (width 0.25) (layer B.Cu) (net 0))
 (segment (start 151.2312 97.391) (end 151.2312 95.859) (width 0.25) (layer F.Cu) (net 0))
 (segment (start 156 100.3046) (end 154.1448 100.3046) (width 0.25) (layer F.Cu) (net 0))
 (segment (start 154.1448 100.3046) (end 151.2312 97.391) (width 0.25) (layer F.Cu) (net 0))
 (via (at 146.0754 95.5802) (size 0.8) (drill 0.4) (layers F.Cu B.Cu) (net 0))
 (segment (start 148.971 95.5746) (end 146.081 95.5746) (width 0.25) (layer B.Cu) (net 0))
 (segment (start 146.081 95.5746) (end 146.0754 95.5802) (width 0.25) (layer B.Cu) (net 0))
 (segment (start 146.0754 95.5802) (end 146.7358 96.2406) (width 0.25) (layer F.Cu) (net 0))
 (segment (start 146.7358 96.2406) (end 146.7358 96.9264) (width 0.25) (layer F.Cu) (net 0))
 (segment (start 146.7358 96.9264) (end 146.9898 97.1804) (width 0.25) (layer F.Cu) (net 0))
 (segment (start 148.0312 96.159) (end 148.0312 95.859) (width 0.25) (layer F.Cu) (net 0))
 (segment (start 147.0098 97.1804) (end 148.0312 96.159) (width 0.25) (layer F.Cu) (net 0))
 (segment (start 146.9898 97.1804) (end 147.0098 97.1804) (width 0.25) (layer F.Cu) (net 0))
 (segment (start 148.971 93.5746) (end 146.7602 93.5746) (width 0.25) (layer B.Cu) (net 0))
 (via (at 144.8816 95.4786) (size 0.8) (drill 0.4) (layers F.Cu B.Cu) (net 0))
 (segment (start 146.7602 93.5746) (end 144.8816 95.4532) (width 0.25) (layer B.Cu) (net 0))
 (segment (start 144.8816 95.4532) (end 144.8816 95.4786) (width 0.25) (layer B.Cu) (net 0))
 (segment (start 144.8816 95.4786) (end 145.9484 96.5454) (width 0.25) (layer F.Cu) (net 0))
 (segment (start 145.9484 96.5454) (end 145.9484 96.9772) (width 0.25) (layer F.Cu) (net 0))
 (segment (start 145.9484 96.9772) (end 146.8374 97.8662) (width 0.25) (layer F.Cu) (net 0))
 (segment (start 146.8374 97.8662) (end 149.2758 97.8662) (width 0.25) (layer F.Cu) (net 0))
 (segment (start 149.6312 97.5108) (end 149.6312 95.859) (width 0.25) (layer F.Cu) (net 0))
 (segment (start 149.2758 97.8662) (end 149.6312 97.5108) (width 0.25) (layer F.Cu) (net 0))
 (via (at 141.2878 98.8316) (size 0.8) (drill 0.4) (layers F.Cu B.Cu) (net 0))
 (segment (start 145.478 98.8316) (end 148.221 101.5746) (width 0.25) (layer B.Cu) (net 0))
 (segment (start 148.221 101.5746) (end 148.971 101.5746) (width 0.25) (layer B.Cu) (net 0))
 (segment (start 141.2878 98.8316) (end 145.478 98.8316) (width 0.25) (layer B.Cu) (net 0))
 (segment (start 141.2878 98.3566) (end 141.3002 98.3442) (width 0.25) (layer B.Cu) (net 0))
 (segment (start 141.2878 98.8316) (end 141.2878 98.3566) (width 0.25) (layer B.Cu) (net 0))
 (segment (start 141.3002 98.3442) (end 141.3002 95.3262) (width 0.25) (layer B.Cu) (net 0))
 (segment (start 145.0518 91.5746) (end 148.971 91.5746) (width 0.25) (layer B.Cu) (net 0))
 (segment (start 141.3002 95.3262) (end 145.0518 91.5746) (width 0.25) (layer B.Cu) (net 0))
 (segment (start 140.4366 84.6328) (end 140.4747 84.5947) (width 0.25) (layer F.Cu) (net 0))
 (segment (start 125.3744 84.6328) (end 140.4366 84.6328) (width 0.25) (layer F.Cu) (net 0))
 (segment (start 124.4854 85.5218) (end 125.3744 84.6328) (width 0.25) (layer F.Cu) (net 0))
 (segment (start 140.4747 84.5947) (end 140.4747 82.38236) (width 0.25) (layer F.Cu) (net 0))
 (segment (start 126.1364 92.3544) (end 124.4854 92.3544) (width 0.25) (layer F.Cu) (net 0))
 (segment (start 124.4854 92.3544) (end 124.4854 85.5218) (width 0.25) (layer F.Cu) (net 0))
 (segment (start 139.573 93.345) (end 139.573 92.1766) (width 0.25) (layer F.Cu) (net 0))
 (segment (start 139.573 88.392) (end 139.72 88.539) (width 0.25) (layer F.Cu) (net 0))
 (segment (start 139.72 88.539) (end 141.498 88.539) (width 0.25) (layer F.Cu) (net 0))
 (segment (start 139.573 88.392) (end 139.573 87.8078) (width 0.25) (layer F.Cu) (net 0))
 (segment (start 142.998 86.237) (end 142.998 88.239) (width 0.25) (layer F.Cu) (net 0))
 (segment (start 156.0322 84.9376) (end 144.2974 84.9376) (width 0.25) (layer F.Cu) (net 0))
 (segment (start 144.2974 84.9376) (end 142.998 86.237) (width 0.25) (layer F.Cu) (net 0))
 (segment (start 142.42034 83.30546) (end 142.42034 84.35594) (width 0.25) (layer F.Cu) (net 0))
 (via (at 142.7988 84.7344) (size 0.8) (drill 0.4) (layers F.Cu B.Cu) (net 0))
 (segment (start 142.42034 84.35594) (end 142.7988 84.7344) (width 0.25) (layer F.Cu) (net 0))
 (via (at 141.732 85.7758) (size 0.8) (drill 0.4) (layers F.Cu B.Cu) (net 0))
 (segment (start 142.7988 84.7344) (end 142.7734 84.7344) (width 0.25) (layer B.Cu) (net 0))
 (segment (start 142.7734 84.7344) (end 141.732 85.7758) (width 0.25) (layer B.Cu) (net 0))
 (segment (start 141.732 85.7758) (end 141.732 86.6902) (width 0.25) (layer F.Cu) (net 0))
 (segment (start 141.998 86.9562) (end 141.998 88.239) (width 0.25) (layer F.Cu) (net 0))
 (segment (start 141.732 86.6902) (end 141.998 86.9562) (width 0.25) (layer F.Cu) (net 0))
 (via (at 145.4658 89.5858) (size 0.8) (drill 0.4) (layers F.Cu B.Cu) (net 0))
 (segment (start 144.8196 89.5746) (end 145.4546 89.5746) (width 0.25) (layer B.Cu) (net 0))
 (segment (start 145.4546 89.5746) (end 145.4658 89.5858) (width 0.25) (layer B.Cu) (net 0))
 (segment (start 145.4658 89.5858) (end 145.4912 89.6112) (width 0.25) (layer F.Cu) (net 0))
 (segment (start 145.4912 89.6112) (end 145.4912 89.9668) (width 0.25) (layer F.Cu) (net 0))
 (segment (start 145.419 90.039) (end 144.298 90.039) (width 0.25) (layer F.Cu) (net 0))
 (segment (start 145.4912 89.9668) (end 145.419 90.039) (width 0.25) (layer F.Cu) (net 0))
 (segment (start 143.861 87.5746) (end 144.6738 87.5746) (width 0.25) (layer B.Cu) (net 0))
 (segment (start 144.6738 87.5746) (end 146.2024 89.1032) (width 0.25) (layer B.Cu) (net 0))
 (segment (start 146.2024 89.1032) (end 146.2024 90.3732) (width 0.25) (layer B.Cu) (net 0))
 (via (at 146.2024 90.3732) (size 0.8) (drill 0.4) (layers F.Cu B.Cu) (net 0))
 (segment (start 146.2024 90.3732) (end 145.7198 90.8558) (width 0.25) (layer F.Cu) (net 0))
 (segment (start 145.403 90.539) (end 144.298 90.539) (width 0.25) (layer F.Cu) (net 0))
 (segment (start 145.7198 90.8558) (end 145.403 90.539) (width 0.25) (layer F.Cu) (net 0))
 (segment (start 140.3858 101.6808) (end 140.3858 92.7354) (width 0.25) (layer B.Cu) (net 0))
 (segment (start 142.143 101.6808) (end 140.3858 101.6808) (width 0.25) (layer B.Cu) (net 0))
 (segment (start 140.3858 101.6808) (end 135.9408 101.6808) (width 0.25) (layer B.Cu) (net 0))
 (via (at 140.589 92.5322) (size 0.8) (drill 0.4) (layers F.Cu B.Cu) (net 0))
 (segment (start 140.3858 92.7354) (end 140.589 92.5322) (width 0.25) (layer B.Cu) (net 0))
 (segment (start 140.589 92.5322) (end 141.478 92.5322) (width 0.25) (layer F.Cu) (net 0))
 (segment (start 141.478 92.5322) (end 141.8082 92.202) (width 0.25) (layer F.Cu) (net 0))
 (segment (start 141.835 92.202) (end 141.998 92.039) (width 0.25) (layer F.Cu) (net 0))
 (segment (start 141.998 92.039) (end 141.998 91.339) (width 0.25) (layer F.Cu) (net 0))
 (segment (start 141.8082 92.202) (end 141.835 92.202) (width 0.25) (layer F.Cu) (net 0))
 (segment (start 139.573 88.9762) (end 139.573 88.392) (width 0.25) (layer F.Cu) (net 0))
 (segment (start 140.4686 89.5096) (end 139.573 89.5096) (width 0.25) (layer F.Cu) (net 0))
 (segment (start 140.498 89.539) (end 140.4686 89.5096) (width 0.25) (layer F.Cu) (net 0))
 (segment (start 141.198 89.539) (end 140.498 89.539) (width 0.25) (layer F.Cu) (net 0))
 (segment (start 139.573 92.1766) (end 139.573 89.5096) (width 0.25) (layer F.Cu) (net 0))
 (segment (start 139.573 89.5096) (end 139.573 88.9762) (width 0.25) (layer F.Cu) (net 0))
 (segment (start 145.0848 103.877719) (end 145.0594 103.852319) (width 0.25) (layer F.Cu) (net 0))
 (segment (start 145.0848 105.0798) (end 145.0848 103.877719) (width 0.25) (layer F.Cu) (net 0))
 (segment (start 145.0594 103.852319) (end 145.0594 103.2002) (width 0.25) (layer F.Cu) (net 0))
 (segment (start 145.0594 103.2002) (end 140.5128 103.2002) (width 0.25) (layer F.Cu) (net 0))
 (via (at 139.7254 102.6414) (size 0.8) (drill 0.4) (layers F.Cu B.Cu) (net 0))
 (segment (start 140.5128 103.2002) (end 140.2842 103.2002) (width 0.25) (layer F.Cu) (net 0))
 (segment (start 140.2842 103.2002) (end 139.7254 102.6414) (width 0.25) (layer F.Cu) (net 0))
 (segment (start 144.8816 94.6912) (end 139.573 94.6912) (width 0.25) (layer F.Cu) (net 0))
 (segment (start 146.812 92.7608) (end 144.8816 94.6912) (width 0.25) (layer F.Cu) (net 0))
 (segment (start 146.812 89.5096) (end 146.812 92.7608) (width 0.25) (layer F.Cu) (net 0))
 (segment (start 139.573 94.6912) (end 139.573 93.345) (width 0.25) (layer F.Cu) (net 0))
 (segment (start 148.0312 91.059) (end 148.0312 89.535) (width 0.25) (layer F.Cu) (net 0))
 (segment (start 147.0152 89.3064) (end 146.812 89.5096) (width 0.25) (layer F.Cu) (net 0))
 (segment (start 139.573 97.1042) (end 139.573 94.6912) (width 0.25) (layer F.Cu) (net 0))
 (segment (start 148.0312 89.535) (end 147.8026 89.3064) (width 0.25) (layer F.Cu) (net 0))
 (segment (start 147.8026 89.3064) (end 147.0152 89.3064) (width 0.25) (layer F.Cu) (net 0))
 (segment (start 144.2212 91.2622) (end 143.998 91.039) (width 0.25) (layer F.Cu) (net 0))
 (segment (start 144.2212 93.3704) (end 144.2212 91.2622) (width 0.25) (layer F.Cu) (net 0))
 (via (at 135.4836 102.6668) (size 0.8) (drill 0.4) (layers F.Cu B.Cu) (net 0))
 (segment (start 139.7254 102.6414) (end 135.509 102.6414) (width 0.25) (layer B.Cu) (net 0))
 (segment (start 135.509 102.6414) (end 135.4836 102.6668) (width 0.25) (layer B.Cu) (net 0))
 (via (at 135.7376 92.1766) (size 0.8) (drill 0.4) (layers F.Cu B.Cu) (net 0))
 (segment (start 135.4836 102.6668) (end 135.4836 92.4306) (width 0.25) (layer F.Cu) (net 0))
 (segment (start 135.4836 92.4306) (end 135.7376 92.1766) (width 0.25) (layer F.Cu) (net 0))
 (segment (start 135.1356 91.5746) (end 133.571 91.5746) (width 0.25) (layer B.Cu) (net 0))
 (segment (start 135.7376 92.1766) (end 135.1356 91.5746) (width 0.25) (layer B.Cu) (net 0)))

